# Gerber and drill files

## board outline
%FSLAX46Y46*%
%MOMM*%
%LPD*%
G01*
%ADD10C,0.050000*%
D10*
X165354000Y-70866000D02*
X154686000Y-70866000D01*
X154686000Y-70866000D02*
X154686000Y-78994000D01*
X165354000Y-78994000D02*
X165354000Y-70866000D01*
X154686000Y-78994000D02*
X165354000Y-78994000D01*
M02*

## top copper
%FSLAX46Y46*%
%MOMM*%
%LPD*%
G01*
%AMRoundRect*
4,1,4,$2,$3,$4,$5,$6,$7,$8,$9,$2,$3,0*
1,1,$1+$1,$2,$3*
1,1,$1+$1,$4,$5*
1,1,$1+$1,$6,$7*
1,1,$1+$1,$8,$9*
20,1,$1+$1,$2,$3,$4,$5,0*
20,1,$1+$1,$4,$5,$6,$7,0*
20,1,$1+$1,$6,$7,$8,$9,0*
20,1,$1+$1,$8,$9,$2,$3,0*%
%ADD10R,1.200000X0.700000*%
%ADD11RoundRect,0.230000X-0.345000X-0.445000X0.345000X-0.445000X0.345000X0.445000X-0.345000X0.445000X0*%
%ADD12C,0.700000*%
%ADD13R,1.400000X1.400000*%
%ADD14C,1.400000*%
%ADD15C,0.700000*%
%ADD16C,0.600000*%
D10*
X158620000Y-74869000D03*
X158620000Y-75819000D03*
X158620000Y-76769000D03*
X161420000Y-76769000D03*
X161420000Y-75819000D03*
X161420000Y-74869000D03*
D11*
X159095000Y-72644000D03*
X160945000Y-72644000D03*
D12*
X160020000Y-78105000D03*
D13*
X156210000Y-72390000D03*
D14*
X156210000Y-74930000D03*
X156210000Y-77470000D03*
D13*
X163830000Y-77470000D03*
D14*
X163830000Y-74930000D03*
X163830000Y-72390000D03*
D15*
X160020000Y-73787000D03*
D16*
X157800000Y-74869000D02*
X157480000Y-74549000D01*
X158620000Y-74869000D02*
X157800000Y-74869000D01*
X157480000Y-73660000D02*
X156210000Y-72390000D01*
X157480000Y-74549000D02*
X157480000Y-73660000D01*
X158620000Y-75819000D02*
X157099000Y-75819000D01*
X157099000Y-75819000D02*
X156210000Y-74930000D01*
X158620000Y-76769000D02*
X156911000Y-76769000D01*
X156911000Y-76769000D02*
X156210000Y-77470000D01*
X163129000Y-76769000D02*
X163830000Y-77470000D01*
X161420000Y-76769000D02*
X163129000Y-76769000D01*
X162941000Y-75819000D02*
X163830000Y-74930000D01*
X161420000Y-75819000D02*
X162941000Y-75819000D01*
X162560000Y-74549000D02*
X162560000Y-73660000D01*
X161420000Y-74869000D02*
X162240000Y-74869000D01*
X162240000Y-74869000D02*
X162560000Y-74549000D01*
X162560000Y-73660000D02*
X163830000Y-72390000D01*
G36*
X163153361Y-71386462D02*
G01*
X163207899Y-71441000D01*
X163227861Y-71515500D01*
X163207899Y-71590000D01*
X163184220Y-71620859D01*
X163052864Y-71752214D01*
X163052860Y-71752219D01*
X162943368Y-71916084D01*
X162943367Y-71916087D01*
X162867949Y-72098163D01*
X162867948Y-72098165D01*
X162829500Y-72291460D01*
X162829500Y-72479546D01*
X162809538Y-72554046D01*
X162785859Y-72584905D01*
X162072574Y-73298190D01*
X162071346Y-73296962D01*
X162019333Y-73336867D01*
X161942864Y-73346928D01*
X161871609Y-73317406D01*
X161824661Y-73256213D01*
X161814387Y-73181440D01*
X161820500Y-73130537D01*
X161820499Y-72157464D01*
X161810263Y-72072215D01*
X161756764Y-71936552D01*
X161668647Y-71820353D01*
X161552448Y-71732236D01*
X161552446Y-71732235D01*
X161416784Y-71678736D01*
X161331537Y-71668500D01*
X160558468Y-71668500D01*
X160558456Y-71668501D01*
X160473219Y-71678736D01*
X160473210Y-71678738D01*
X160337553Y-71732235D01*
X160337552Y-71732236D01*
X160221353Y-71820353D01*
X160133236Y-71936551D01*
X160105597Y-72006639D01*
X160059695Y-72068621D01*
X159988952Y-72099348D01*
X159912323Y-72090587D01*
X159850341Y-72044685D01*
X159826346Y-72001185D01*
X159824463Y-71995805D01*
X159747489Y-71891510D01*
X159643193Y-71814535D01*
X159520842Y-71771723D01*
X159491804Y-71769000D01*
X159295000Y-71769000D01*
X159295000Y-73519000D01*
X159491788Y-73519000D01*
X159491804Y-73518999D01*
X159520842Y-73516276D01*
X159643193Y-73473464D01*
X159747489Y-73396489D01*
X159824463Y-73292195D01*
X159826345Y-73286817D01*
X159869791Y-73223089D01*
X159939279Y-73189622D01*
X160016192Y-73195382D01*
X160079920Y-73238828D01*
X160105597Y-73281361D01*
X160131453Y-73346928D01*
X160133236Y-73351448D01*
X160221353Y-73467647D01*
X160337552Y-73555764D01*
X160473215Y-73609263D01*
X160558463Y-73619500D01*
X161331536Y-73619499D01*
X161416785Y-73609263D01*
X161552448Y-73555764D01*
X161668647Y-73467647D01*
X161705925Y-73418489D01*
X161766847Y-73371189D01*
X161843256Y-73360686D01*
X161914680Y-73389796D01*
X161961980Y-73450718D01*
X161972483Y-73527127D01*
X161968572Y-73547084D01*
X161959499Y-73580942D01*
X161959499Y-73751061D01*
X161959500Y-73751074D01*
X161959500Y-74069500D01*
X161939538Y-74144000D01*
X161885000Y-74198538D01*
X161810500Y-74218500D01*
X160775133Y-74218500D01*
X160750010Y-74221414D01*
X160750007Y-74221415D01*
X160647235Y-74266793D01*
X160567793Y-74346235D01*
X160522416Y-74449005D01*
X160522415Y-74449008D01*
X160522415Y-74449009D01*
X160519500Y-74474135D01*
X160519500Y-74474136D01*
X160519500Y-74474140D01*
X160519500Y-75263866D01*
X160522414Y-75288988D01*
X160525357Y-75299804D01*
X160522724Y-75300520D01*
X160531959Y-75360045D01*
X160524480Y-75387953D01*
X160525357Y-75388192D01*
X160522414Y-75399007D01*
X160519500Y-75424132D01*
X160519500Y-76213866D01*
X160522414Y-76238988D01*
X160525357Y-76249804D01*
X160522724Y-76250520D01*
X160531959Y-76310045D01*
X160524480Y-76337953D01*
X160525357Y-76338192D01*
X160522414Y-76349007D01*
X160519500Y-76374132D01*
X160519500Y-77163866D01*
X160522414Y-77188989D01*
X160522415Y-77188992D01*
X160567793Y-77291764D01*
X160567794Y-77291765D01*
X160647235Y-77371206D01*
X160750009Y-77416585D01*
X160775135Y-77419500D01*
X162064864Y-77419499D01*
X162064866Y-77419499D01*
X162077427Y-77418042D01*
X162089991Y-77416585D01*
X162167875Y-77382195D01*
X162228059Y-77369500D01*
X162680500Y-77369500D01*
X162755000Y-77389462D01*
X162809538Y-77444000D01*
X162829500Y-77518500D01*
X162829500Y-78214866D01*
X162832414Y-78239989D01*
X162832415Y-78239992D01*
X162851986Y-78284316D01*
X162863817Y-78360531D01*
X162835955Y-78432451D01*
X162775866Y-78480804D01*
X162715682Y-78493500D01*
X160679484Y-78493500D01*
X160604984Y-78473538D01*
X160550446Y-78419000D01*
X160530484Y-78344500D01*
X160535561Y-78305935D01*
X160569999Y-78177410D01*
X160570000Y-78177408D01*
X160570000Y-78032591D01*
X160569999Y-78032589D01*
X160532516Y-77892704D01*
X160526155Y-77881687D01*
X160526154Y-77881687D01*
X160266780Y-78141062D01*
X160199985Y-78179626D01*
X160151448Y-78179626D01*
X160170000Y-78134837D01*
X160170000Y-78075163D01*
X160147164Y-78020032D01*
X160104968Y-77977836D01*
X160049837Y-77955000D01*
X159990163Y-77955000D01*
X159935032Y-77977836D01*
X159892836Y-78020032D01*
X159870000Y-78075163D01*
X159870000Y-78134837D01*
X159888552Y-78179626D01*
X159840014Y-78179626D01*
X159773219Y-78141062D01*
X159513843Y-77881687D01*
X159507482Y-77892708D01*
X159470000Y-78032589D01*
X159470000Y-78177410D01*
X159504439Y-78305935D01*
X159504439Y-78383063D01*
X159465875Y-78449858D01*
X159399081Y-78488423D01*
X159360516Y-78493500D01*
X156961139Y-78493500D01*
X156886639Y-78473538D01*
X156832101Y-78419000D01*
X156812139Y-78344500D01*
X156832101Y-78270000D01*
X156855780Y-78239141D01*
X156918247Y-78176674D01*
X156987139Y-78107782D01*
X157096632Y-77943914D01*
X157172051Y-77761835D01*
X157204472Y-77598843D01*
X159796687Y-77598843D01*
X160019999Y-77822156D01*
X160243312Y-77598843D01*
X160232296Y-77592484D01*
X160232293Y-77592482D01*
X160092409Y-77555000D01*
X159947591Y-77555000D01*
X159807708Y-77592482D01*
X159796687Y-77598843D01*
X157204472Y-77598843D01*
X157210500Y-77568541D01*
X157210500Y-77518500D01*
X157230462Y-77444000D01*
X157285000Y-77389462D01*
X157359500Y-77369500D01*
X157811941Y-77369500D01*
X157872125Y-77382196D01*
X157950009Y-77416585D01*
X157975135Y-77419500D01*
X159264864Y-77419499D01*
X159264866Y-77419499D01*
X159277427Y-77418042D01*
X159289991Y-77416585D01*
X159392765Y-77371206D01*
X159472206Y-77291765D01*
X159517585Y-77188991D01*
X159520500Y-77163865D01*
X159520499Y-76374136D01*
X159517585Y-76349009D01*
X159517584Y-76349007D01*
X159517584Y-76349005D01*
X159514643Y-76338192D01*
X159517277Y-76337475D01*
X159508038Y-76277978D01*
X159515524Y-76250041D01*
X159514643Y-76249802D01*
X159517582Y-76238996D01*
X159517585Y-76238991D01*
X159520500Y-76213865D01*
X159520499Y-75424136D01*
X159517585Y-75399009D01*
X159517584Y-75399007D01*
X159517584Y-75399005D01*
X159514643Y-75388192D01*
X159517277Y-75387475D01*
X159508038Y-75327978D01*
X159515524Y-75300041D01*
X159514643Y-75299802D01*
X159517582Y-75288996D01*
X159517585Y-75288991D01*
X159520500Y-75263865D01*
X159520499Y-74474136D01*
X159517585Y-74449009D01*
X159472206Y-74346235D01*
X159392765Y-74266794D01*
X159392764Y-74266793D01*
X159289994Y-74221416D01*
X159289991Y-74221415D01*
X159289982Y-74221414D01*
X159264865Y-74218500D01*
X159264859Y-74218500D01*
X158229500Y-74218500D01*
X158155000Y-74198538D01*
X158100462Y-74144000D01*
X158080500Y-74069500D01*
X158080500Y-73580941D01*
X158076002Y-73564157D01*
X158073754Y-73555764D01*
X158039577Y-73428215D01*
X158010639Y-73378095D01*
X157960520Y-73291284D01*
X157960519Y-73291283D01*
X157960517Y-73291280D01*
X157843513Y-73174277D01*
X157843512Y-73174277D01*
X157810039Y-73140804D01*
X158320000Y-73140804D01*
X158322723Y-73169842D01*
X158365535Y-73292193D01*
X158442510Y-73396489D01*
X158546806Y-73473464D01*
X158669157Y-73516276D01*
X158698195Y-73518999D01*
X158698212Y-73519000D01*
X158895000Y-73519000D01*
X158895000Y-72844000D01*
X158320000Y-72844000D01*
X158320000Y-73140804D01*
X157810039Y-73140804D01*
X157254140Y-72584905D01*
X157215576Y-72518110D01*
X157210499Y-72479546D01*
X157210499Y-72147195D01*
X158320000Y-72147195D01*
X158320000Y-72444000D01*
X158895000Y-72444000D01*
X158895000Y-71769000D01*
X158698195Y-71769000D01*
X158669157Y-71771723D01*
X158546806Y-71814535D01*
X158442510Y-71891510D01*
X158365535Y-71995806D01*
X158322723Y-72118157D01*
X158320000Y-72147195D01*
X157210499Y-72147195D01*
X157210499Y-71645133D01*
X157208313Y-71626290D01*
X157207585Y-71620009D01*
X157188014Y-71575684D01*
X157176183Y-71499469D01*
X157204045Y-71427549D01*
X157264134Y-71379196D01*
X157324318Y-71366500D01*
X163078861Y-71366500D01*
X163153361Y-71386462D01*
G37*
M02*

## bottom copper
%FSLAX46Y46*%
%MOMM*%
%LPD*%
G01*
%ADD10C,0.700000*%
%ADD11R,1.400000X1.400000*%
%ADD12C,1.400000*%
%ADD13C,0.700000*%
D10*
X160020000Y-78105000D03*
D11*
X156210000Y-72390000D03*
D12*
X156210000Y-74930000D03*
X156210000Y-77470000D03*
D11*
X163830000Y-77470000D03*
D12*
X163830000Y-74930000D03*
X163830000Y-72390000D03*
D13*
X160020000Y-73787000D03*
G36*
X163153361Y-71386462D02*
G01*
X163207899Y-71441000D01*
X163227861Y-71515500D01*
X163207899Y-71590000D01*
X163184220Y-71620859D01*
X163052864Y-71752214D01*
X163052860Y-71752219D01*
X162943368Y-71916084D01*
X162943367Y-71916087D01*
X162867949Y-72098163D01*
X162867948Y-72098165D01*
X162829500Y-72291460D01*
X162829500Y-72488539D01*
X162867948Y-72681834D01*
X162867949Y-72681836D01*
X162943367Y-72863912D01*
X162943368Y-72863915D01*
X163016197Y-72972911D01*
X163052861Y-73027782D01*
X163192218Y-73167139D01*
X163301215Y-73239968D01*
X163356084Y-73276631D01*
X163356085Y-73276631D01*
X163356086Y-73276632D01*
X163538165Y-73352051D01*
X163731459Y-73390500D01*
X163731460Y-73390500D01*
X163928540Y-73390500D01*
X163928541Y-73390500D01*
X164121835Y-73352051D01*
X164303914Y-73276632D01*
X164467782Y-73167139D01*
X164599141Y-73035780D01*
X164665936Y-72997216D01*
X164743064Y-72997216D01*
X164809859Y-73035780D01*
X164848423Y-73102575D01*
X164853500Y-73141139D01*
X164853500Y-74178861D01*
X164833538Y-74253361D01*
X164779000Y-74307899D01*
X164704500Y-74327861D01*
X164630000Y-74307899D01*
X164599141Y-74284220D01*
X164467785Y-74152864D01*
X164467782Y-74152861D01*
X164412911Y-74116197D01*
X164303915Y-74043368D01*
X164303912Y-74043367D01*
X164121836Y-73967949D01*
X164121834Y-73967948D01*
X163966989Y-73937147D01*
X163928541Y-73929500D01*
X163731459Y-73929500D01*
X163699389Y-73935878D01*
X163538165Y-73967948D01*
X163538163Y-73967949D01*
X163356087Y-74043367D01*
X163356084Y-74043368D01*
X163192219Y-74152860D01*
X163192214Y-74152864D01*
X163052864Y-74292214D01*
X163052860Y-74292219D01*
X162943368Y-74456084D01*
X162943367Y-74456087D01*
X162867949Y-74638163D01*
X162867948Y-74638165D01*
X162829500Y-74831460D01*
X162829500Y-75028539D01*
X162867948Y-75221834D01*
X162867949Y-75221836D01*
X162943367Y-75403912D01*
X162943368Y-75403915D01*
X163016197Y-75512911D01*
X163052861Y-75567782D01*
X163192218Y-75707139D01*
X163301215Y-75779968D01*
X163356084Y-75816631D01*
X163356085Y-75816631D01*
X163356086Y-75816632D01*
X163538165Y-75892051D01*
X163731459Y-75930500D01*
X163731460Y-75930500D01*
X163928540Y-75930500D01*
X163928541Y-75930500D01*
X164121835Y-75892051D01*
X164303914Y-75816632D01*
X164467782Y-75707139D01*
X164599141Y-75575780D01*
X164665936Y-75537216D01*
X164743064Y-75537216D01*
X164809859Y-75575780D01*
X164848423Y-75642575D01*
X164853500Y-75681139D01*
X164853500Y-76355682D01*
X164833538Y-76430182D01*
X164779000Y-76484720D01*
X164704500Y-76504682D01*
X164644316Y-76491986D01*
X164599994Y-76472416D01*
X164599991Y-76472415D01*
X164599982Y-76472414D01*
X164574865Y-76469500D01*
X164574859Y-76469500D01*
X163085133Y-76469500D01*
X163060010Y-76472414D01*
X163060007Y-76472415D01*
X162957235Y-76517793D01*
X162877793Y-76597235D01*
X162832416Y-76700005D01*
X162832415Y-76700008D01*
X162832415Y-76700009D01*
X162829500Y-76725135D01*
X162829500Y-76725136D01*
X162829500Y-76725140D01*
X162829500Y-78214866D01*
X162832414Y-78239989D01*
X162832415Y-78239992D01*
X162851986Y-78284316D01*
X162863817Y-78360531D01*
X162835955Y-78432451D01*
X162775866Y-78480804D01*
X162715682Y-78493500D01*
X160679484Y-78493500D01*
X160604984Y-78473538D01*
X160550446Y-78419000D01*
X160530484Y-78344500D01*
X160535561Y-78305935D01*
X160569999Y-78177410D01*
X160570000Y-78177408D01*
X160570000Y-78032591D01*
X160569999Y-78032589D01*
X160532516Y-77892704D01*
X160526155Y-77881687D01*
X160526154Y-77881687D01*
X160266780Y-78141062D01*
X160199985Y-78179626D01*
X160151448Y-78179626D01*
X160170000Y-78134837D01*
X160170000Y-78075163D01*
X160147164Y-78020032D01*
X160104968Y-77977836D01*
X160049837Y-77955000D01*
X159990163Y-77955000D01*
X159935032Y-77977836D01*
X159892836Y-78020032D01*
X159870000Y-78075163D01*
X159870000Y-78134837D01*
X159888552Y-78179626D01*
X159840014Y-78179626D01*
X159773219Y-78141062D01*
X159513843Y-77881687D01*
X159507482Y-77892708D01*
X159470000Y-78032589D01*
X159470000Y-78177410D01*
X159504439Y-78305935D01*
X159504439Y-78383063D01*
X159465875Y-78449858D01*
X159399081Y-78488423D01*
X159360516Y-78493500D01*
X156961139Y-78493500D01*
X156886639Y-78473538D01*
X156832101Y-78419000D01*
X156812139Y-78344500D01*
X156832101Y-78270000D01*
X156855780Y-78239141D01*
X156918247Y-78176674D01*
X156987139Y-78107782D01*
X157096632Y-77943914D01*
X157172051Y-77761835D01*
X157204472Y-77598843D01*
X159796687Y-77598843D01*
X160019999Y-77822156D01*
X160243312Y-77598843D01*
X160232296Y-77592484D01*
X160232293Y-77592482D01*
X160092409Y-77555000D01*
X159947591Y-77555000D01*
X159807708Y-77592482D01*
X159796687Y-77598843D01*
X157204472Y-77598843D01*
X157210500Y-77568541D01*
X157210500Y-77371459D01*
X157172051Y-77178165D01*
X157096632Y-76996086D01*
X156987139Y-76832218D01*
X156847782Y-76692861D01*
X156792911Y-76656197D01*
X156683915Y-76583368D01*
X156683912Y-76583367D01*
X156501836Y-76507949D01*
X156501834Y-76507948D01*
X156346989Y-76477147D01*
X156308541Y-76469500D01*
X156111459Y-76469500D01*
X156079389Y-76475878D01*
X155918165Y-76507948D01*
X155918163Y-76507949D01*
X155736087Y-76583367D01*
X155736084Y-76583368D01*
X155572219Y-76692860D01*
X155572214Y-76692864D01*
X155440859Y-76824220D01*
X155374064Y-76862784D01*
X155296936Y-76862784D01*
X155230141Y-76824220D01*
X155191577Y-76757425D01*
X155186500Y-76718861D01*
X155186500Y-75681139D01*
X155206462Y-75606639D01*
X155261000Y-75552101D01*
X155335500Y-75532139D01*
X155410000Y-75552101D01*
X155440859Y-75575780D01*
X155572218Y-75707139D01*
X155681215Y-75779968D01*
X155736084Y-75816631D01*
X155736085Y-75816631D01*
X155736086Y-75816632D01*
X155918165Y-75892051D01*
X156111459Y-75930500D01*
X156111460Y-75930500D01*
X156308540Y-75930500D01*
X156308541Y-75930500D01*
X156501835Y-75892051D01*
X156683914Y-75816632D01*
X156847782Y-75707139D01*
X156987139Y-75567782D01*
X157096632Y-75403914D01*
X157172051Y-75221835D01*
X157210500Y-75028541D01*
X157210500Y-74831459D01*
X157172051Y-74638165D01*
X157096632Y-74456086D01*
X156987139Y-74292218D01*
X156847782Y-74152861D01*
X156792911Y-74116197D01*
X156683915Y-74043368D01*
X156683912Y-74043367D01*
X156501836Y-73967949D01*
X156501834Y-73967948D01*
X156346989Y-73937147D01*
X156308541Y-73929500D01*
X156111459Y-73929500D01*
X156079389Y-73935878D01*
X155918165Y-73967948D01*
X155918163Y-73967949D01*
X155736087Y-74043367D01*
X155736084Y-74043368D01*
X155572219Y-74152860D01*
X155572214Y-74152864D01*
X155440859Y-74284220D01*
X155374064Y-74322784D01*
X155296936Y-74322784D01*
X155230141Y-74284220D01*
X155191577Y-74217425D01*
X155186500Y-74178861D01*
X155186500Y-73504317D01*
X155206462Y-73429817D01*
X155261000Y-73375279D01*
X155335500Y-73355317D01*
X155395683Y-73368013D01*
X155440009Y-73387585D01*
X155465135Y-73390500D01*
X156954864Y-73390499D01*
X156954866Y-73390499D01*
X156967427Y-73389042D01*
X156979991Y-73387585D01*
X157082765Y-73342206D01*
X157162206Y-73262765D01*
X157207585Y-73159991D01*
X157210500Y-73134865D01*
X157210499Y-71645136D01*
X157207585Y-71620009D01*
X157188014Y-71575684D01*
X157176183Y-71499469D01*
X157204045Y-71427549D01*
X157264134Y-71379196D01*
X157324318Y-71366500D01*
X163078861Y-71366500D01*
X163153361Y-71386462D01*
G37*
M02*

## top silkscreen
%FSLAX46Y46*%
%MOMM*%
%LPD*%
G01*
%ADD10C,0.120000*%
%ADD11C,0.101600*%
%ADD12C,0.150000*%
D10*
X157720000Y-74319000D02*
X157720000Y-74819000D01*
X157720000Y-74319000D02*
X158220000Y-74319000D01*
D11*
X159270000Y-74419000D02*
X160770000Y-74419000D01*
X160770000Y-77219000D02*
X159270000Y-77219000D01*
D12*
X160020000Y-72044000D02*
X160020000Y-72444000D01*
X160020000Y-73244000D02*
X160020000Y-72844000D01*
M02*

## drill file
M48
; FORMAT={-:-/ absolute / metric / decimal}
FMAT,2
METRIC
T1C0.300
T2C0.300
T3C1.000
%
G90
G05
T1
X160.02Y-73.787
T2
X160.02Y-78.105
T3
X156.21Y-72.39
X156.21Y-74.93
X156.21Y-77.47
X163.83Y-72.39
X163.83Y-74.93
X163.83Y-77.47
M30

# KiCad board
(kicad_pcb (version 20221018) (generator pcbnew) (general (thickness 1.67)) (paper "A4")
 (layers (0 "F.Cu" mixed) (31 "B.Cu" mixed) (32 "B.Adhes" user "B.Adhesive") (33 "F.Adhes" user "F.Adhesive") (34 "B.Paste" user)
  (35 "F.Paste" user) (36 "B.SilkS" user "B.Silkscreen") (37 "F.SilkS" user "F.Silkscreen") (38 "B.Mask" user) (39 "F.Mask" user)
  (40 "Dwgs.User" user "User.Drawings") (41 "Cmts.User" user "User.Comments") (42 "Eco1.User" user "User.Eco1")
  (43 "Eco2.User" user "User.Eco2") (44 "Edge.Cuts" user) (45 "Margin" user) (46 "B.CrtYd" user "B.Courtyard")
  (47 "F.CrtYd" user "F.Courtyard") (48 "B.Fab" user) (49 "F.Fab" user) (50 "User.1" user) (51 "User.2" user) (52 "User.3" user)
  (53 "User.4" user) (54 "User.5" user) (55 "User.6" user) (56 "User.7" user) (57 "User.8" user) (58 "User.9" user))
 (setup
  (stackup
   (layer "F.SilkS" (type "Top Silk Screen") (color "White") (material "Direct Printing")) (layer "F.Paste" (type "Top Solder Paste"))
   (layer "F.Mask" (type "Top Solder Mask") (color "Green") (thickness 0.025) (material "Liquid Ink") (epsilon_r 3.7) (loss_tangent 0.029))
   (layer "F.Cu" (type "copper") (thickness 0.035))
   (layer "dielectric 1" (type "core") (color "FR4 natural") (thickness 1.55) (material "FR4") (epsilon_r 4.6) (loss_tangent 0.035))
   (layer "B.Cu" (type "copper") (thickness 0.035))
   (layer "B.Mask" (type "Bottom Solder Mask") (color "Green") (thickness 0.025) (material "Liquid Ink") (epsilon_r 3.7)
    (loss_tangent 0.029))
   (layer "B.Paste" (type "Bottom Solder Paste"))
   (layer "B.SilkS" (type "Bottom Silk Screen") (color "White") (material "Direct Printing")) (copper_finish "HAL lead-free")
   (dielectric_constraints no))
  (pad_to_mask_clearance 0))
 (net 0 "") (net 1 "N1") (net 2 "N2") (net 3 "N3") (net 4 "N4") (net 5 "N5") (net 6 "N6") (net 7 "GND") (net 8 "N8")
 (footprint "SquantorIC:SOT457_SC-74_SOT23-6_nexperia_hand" (layer "F.Cu") (at 160.02 75.819)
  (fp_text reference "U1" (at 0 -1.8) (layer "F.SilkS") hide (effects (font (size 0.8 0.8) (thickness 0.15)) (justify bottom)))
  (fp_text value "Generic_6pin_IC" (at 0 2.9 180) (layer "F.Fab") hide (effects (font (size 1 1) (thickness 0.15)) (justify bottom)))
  (fp_line (start -2.3 -1.5) (end -2.3 -1) (stroke (width 0.12) (type solid)) (layer "F.SilkS"))
  (fp_line (start -2.3 -1.5) (end -1.8 -1.5) (stroke (width 0.12) (type solid)) (layer "F.SilkS"))
  (fp_line (start -0.75 -1.4) (end 0.75 -1.4) (stroke (width 0.1016) (type solid)) (layer "F.SilkS"))
  (fp_line (start 0.75 1.4) (end -0.75 1.4) (stroke (width 0.1016) (type solid)) (layer "F.SilkS"))
  (pad "1" smd rect (at -1.4 -0.95 270) (size 0.7 1.2) (layers "F.Cu" "F.Paste" "F.Mask") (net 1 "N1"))
  (pad "2" smd rect (at -1.4 0 270) (size 0.7 1.2) (layers "F.Cu" "F.Paste" "F.Mask") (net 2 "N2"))
  (pad "3" smd rect (at -1.4 0.95 270) (size 0.7 1.2) (layers "F.Cu" "F.Paste" "F.Mask") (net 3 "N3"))
  (pad "4" smd rect (at 1.4 0.95 270) (size 0.7 1.2) (layers "F.Cu" "F.Paste" "F.Mask") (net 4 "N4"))
  (pad "5" smd rect (at 1.4 0 270) (size 0.7 1.2) (layers "F.Cu" "F.Paste" "F.Mask") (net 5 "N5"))
  (pad "6" smd rect (at 1.4 -0.95 270) (size 0.7 1.2) (layers "F.Cu" "F.Paste" "F.Mask") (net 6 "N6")))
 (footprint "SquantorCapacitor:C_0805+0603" (layer "F.Cu") (at 160.02 72.644)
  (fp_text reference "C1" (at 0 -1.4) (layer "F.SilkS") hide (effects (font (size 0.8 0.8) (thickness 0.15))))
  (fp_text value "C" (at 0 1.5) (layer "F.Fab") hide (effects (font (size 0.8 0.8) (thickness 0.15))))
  (fp_line (start 0 -0.6) (end 0 -0.2) (stroke (width 0.15) (type solid)) (layer "F.SilkS"))
  (fp_line (start 0 0.6) (end 0 0.2) (stroke (width 0.15) (type solid)) (layer "F.SilkS"))
  (pad "1" smd roundrect (at -0.925 0) (size 1.15 1.35) (layers "F.Cu" "F.Paste" "F.Mask") (roundrect_rratio 0.2) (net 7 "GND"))
  (pad "2" smd roundrect (at 0.925 0) (size 1.15 1.35) (layers "F.Cu" "F.Paste" "F.Mask") (roundrect_rratio 0.2) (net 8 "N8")))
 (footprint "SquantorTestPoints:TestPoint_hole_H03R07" (layer "F.Cu") (at 160.02 78.105)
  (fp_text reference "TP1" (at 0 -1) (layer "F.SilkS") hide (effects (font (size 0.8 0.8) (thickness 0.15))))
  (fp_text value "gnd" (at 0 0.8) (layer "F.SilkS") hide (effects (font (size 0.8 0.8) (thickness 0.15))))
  (pad "1" thru_hole circle (at 0 0) (size 0.7 0.7) (drill 0.3) (layers "*.Cu" "*.Mask") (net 7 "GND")))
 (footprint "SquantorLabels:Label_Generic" (layer "B.Cu") (at 160.02 74.295 -90)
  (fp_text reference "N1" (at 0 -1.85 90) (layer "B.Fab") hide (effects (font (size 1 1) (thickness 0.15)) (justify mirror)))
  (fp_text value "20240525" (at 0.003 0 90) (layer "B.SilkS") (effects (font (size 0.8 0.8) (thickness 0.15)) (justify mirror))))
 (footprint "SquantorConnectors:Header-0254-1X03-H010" (layer "B.Cu") (at 156.21 74.93 -90)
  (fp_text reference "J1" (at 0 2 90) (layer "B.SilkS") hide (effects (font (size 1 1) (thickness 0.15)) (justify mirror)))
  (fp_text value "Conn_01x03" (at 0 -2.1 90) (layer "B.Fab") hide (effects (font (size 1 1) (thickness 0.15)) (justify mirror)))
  (pad "1" thru_hole rect (at -2.54 0 90) (size 1.4 1.4) (drill 1) (layers "*.Cu" "*.Mask") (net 1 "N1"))
  (pad "2" thru_hole circle (at 0 0 90) (size 1.4 1.4) (drill 1) (layers "*.Cu" "*.Mask") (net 2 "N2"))
  (pad "3" thru_hole circle (at 2.54 0 90) (size 1.4 1.4) (drill 1) (layers "*.Cu" "*.Mask") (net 3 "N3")))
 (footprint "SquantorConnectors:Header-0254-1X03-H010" (layer "B.Cu") (at 163.83 74.93 90)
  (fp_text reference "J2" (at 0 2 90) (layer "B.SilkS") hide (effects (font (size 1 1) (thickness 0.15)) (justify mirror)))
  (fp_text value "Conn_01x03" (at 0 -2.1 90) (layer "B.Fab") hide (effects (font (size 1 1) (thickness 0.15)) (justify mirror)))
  (pad "1" thru_hole rect (at -2.54 0 270) (size 1.4 1.4) (drill 1) (layers "*.Cu" "*.Mask") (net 4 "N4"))
  (pad "2" thru_hole circle (at 0 0 270) (size 1.4 1.4) (drill 1) (layers "*.Cu" "*.Mask") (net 5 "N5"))
  (pad "3" thru_hole circle (at 2.54 0 270) (size 1.4 1.4) (drill 1) (layers "*.Cu" "*.Mask") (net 6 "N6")))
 (gr_line (start 165.354 70.866) (end 154.686 70.866) (stroke (width 0.05) (type solid)) (layer "Edge.Cuts"))
 (gr_line (start 154.686 70.866) (end 154.686 78.994) (stroke (width 0.05) (type solid)) (layer "Edge.Cuts"))
 (gr_line (start 165.354 78.994) (end 165.354 70.866) (stroke (width 0.05) (type solid)) (layer "Edge.Cuts"))
 (gr_line (start 154.686 78.994) (end 165.354 78.994) (stroke (width 0.05) (type solid)) (layer "Edge.Cuts"))
 (via (at 160.02 73.787) (size 0.7) (drill 0.3) (layers "F.Cu" "B.Cu") (free) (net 7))
 (segment (start 157.8 74.869) (end 157.48 74.549) (width 0.6) (layer "F.Cu") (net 1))
 (segment (start 158.62 74.869) (end 157.8 74.869) (width 0.6) (layer "F.Cu") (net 1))
 (segment (start 157.48 73.66) (end 156.21 72.39) (width 0.6) (layer "F.Cu") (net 1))
 (segment (start 157.48 74.549) (end 157.48 73.66) (width 0.6) (layer "F.Cu") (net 1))
 (segment (start 158.62 75.819) (end 157.099 75.819) (width 0.6) (layer "F.Cu") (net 2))
 (segment (start 157.099 75.819) (end 156.21 74.93) (width 0.6) (layer "F.Cu") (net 2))
 (segment (start 158.62 76.769) (end 156.911 76.769) (width 0.6) (layer "F.Cu") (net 3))
 (segment (start 156.911 76.769) (end 156.21 77.47) (width 0.6) (layer "F.Cu") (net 3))
 (segment (start 163.129 76.769) (end 163.83 77.47) (width 0.6) (layer "F.Cu") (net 4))
 (segment (start 161.42 76.769) (end 163.129 76.769) (width 0.6) (layer "F.Cu") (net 4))
 (segment (start 162.941 75.819) (end 163.83 74.93) (width 0.6) (layer "F.Cu") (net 5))
 (segment (start 161.42 75.819) (end 162.941 75.819) (width 0.6) (layer "F.Cu") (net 5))
 (segment (start 162.56 74.549) (end 162.56 73.66) (width 0.6) (layer "F.Cu") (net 6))
 (segment (start 161.42 74.869) (end 162.24 74.869) (width 0.6) (layer "F.Cu") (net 6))
 (segment (start 162.24 74.869) (end 162.56 74.549) (width 0.6) (layer "F.Cu") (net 6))
 (segment (start 162.56 73.66) (end 163.83 72.39) (width 0.6) (layer "F.Cu") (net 6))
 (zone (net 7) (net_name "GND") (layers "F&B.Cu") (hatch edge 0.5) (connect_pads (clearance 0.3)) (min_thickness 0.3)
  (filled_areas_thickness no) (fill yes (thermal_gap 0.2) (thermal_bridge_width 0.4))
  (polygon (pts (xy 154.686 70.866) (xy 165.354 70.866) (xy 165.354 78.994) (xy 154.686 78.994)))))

